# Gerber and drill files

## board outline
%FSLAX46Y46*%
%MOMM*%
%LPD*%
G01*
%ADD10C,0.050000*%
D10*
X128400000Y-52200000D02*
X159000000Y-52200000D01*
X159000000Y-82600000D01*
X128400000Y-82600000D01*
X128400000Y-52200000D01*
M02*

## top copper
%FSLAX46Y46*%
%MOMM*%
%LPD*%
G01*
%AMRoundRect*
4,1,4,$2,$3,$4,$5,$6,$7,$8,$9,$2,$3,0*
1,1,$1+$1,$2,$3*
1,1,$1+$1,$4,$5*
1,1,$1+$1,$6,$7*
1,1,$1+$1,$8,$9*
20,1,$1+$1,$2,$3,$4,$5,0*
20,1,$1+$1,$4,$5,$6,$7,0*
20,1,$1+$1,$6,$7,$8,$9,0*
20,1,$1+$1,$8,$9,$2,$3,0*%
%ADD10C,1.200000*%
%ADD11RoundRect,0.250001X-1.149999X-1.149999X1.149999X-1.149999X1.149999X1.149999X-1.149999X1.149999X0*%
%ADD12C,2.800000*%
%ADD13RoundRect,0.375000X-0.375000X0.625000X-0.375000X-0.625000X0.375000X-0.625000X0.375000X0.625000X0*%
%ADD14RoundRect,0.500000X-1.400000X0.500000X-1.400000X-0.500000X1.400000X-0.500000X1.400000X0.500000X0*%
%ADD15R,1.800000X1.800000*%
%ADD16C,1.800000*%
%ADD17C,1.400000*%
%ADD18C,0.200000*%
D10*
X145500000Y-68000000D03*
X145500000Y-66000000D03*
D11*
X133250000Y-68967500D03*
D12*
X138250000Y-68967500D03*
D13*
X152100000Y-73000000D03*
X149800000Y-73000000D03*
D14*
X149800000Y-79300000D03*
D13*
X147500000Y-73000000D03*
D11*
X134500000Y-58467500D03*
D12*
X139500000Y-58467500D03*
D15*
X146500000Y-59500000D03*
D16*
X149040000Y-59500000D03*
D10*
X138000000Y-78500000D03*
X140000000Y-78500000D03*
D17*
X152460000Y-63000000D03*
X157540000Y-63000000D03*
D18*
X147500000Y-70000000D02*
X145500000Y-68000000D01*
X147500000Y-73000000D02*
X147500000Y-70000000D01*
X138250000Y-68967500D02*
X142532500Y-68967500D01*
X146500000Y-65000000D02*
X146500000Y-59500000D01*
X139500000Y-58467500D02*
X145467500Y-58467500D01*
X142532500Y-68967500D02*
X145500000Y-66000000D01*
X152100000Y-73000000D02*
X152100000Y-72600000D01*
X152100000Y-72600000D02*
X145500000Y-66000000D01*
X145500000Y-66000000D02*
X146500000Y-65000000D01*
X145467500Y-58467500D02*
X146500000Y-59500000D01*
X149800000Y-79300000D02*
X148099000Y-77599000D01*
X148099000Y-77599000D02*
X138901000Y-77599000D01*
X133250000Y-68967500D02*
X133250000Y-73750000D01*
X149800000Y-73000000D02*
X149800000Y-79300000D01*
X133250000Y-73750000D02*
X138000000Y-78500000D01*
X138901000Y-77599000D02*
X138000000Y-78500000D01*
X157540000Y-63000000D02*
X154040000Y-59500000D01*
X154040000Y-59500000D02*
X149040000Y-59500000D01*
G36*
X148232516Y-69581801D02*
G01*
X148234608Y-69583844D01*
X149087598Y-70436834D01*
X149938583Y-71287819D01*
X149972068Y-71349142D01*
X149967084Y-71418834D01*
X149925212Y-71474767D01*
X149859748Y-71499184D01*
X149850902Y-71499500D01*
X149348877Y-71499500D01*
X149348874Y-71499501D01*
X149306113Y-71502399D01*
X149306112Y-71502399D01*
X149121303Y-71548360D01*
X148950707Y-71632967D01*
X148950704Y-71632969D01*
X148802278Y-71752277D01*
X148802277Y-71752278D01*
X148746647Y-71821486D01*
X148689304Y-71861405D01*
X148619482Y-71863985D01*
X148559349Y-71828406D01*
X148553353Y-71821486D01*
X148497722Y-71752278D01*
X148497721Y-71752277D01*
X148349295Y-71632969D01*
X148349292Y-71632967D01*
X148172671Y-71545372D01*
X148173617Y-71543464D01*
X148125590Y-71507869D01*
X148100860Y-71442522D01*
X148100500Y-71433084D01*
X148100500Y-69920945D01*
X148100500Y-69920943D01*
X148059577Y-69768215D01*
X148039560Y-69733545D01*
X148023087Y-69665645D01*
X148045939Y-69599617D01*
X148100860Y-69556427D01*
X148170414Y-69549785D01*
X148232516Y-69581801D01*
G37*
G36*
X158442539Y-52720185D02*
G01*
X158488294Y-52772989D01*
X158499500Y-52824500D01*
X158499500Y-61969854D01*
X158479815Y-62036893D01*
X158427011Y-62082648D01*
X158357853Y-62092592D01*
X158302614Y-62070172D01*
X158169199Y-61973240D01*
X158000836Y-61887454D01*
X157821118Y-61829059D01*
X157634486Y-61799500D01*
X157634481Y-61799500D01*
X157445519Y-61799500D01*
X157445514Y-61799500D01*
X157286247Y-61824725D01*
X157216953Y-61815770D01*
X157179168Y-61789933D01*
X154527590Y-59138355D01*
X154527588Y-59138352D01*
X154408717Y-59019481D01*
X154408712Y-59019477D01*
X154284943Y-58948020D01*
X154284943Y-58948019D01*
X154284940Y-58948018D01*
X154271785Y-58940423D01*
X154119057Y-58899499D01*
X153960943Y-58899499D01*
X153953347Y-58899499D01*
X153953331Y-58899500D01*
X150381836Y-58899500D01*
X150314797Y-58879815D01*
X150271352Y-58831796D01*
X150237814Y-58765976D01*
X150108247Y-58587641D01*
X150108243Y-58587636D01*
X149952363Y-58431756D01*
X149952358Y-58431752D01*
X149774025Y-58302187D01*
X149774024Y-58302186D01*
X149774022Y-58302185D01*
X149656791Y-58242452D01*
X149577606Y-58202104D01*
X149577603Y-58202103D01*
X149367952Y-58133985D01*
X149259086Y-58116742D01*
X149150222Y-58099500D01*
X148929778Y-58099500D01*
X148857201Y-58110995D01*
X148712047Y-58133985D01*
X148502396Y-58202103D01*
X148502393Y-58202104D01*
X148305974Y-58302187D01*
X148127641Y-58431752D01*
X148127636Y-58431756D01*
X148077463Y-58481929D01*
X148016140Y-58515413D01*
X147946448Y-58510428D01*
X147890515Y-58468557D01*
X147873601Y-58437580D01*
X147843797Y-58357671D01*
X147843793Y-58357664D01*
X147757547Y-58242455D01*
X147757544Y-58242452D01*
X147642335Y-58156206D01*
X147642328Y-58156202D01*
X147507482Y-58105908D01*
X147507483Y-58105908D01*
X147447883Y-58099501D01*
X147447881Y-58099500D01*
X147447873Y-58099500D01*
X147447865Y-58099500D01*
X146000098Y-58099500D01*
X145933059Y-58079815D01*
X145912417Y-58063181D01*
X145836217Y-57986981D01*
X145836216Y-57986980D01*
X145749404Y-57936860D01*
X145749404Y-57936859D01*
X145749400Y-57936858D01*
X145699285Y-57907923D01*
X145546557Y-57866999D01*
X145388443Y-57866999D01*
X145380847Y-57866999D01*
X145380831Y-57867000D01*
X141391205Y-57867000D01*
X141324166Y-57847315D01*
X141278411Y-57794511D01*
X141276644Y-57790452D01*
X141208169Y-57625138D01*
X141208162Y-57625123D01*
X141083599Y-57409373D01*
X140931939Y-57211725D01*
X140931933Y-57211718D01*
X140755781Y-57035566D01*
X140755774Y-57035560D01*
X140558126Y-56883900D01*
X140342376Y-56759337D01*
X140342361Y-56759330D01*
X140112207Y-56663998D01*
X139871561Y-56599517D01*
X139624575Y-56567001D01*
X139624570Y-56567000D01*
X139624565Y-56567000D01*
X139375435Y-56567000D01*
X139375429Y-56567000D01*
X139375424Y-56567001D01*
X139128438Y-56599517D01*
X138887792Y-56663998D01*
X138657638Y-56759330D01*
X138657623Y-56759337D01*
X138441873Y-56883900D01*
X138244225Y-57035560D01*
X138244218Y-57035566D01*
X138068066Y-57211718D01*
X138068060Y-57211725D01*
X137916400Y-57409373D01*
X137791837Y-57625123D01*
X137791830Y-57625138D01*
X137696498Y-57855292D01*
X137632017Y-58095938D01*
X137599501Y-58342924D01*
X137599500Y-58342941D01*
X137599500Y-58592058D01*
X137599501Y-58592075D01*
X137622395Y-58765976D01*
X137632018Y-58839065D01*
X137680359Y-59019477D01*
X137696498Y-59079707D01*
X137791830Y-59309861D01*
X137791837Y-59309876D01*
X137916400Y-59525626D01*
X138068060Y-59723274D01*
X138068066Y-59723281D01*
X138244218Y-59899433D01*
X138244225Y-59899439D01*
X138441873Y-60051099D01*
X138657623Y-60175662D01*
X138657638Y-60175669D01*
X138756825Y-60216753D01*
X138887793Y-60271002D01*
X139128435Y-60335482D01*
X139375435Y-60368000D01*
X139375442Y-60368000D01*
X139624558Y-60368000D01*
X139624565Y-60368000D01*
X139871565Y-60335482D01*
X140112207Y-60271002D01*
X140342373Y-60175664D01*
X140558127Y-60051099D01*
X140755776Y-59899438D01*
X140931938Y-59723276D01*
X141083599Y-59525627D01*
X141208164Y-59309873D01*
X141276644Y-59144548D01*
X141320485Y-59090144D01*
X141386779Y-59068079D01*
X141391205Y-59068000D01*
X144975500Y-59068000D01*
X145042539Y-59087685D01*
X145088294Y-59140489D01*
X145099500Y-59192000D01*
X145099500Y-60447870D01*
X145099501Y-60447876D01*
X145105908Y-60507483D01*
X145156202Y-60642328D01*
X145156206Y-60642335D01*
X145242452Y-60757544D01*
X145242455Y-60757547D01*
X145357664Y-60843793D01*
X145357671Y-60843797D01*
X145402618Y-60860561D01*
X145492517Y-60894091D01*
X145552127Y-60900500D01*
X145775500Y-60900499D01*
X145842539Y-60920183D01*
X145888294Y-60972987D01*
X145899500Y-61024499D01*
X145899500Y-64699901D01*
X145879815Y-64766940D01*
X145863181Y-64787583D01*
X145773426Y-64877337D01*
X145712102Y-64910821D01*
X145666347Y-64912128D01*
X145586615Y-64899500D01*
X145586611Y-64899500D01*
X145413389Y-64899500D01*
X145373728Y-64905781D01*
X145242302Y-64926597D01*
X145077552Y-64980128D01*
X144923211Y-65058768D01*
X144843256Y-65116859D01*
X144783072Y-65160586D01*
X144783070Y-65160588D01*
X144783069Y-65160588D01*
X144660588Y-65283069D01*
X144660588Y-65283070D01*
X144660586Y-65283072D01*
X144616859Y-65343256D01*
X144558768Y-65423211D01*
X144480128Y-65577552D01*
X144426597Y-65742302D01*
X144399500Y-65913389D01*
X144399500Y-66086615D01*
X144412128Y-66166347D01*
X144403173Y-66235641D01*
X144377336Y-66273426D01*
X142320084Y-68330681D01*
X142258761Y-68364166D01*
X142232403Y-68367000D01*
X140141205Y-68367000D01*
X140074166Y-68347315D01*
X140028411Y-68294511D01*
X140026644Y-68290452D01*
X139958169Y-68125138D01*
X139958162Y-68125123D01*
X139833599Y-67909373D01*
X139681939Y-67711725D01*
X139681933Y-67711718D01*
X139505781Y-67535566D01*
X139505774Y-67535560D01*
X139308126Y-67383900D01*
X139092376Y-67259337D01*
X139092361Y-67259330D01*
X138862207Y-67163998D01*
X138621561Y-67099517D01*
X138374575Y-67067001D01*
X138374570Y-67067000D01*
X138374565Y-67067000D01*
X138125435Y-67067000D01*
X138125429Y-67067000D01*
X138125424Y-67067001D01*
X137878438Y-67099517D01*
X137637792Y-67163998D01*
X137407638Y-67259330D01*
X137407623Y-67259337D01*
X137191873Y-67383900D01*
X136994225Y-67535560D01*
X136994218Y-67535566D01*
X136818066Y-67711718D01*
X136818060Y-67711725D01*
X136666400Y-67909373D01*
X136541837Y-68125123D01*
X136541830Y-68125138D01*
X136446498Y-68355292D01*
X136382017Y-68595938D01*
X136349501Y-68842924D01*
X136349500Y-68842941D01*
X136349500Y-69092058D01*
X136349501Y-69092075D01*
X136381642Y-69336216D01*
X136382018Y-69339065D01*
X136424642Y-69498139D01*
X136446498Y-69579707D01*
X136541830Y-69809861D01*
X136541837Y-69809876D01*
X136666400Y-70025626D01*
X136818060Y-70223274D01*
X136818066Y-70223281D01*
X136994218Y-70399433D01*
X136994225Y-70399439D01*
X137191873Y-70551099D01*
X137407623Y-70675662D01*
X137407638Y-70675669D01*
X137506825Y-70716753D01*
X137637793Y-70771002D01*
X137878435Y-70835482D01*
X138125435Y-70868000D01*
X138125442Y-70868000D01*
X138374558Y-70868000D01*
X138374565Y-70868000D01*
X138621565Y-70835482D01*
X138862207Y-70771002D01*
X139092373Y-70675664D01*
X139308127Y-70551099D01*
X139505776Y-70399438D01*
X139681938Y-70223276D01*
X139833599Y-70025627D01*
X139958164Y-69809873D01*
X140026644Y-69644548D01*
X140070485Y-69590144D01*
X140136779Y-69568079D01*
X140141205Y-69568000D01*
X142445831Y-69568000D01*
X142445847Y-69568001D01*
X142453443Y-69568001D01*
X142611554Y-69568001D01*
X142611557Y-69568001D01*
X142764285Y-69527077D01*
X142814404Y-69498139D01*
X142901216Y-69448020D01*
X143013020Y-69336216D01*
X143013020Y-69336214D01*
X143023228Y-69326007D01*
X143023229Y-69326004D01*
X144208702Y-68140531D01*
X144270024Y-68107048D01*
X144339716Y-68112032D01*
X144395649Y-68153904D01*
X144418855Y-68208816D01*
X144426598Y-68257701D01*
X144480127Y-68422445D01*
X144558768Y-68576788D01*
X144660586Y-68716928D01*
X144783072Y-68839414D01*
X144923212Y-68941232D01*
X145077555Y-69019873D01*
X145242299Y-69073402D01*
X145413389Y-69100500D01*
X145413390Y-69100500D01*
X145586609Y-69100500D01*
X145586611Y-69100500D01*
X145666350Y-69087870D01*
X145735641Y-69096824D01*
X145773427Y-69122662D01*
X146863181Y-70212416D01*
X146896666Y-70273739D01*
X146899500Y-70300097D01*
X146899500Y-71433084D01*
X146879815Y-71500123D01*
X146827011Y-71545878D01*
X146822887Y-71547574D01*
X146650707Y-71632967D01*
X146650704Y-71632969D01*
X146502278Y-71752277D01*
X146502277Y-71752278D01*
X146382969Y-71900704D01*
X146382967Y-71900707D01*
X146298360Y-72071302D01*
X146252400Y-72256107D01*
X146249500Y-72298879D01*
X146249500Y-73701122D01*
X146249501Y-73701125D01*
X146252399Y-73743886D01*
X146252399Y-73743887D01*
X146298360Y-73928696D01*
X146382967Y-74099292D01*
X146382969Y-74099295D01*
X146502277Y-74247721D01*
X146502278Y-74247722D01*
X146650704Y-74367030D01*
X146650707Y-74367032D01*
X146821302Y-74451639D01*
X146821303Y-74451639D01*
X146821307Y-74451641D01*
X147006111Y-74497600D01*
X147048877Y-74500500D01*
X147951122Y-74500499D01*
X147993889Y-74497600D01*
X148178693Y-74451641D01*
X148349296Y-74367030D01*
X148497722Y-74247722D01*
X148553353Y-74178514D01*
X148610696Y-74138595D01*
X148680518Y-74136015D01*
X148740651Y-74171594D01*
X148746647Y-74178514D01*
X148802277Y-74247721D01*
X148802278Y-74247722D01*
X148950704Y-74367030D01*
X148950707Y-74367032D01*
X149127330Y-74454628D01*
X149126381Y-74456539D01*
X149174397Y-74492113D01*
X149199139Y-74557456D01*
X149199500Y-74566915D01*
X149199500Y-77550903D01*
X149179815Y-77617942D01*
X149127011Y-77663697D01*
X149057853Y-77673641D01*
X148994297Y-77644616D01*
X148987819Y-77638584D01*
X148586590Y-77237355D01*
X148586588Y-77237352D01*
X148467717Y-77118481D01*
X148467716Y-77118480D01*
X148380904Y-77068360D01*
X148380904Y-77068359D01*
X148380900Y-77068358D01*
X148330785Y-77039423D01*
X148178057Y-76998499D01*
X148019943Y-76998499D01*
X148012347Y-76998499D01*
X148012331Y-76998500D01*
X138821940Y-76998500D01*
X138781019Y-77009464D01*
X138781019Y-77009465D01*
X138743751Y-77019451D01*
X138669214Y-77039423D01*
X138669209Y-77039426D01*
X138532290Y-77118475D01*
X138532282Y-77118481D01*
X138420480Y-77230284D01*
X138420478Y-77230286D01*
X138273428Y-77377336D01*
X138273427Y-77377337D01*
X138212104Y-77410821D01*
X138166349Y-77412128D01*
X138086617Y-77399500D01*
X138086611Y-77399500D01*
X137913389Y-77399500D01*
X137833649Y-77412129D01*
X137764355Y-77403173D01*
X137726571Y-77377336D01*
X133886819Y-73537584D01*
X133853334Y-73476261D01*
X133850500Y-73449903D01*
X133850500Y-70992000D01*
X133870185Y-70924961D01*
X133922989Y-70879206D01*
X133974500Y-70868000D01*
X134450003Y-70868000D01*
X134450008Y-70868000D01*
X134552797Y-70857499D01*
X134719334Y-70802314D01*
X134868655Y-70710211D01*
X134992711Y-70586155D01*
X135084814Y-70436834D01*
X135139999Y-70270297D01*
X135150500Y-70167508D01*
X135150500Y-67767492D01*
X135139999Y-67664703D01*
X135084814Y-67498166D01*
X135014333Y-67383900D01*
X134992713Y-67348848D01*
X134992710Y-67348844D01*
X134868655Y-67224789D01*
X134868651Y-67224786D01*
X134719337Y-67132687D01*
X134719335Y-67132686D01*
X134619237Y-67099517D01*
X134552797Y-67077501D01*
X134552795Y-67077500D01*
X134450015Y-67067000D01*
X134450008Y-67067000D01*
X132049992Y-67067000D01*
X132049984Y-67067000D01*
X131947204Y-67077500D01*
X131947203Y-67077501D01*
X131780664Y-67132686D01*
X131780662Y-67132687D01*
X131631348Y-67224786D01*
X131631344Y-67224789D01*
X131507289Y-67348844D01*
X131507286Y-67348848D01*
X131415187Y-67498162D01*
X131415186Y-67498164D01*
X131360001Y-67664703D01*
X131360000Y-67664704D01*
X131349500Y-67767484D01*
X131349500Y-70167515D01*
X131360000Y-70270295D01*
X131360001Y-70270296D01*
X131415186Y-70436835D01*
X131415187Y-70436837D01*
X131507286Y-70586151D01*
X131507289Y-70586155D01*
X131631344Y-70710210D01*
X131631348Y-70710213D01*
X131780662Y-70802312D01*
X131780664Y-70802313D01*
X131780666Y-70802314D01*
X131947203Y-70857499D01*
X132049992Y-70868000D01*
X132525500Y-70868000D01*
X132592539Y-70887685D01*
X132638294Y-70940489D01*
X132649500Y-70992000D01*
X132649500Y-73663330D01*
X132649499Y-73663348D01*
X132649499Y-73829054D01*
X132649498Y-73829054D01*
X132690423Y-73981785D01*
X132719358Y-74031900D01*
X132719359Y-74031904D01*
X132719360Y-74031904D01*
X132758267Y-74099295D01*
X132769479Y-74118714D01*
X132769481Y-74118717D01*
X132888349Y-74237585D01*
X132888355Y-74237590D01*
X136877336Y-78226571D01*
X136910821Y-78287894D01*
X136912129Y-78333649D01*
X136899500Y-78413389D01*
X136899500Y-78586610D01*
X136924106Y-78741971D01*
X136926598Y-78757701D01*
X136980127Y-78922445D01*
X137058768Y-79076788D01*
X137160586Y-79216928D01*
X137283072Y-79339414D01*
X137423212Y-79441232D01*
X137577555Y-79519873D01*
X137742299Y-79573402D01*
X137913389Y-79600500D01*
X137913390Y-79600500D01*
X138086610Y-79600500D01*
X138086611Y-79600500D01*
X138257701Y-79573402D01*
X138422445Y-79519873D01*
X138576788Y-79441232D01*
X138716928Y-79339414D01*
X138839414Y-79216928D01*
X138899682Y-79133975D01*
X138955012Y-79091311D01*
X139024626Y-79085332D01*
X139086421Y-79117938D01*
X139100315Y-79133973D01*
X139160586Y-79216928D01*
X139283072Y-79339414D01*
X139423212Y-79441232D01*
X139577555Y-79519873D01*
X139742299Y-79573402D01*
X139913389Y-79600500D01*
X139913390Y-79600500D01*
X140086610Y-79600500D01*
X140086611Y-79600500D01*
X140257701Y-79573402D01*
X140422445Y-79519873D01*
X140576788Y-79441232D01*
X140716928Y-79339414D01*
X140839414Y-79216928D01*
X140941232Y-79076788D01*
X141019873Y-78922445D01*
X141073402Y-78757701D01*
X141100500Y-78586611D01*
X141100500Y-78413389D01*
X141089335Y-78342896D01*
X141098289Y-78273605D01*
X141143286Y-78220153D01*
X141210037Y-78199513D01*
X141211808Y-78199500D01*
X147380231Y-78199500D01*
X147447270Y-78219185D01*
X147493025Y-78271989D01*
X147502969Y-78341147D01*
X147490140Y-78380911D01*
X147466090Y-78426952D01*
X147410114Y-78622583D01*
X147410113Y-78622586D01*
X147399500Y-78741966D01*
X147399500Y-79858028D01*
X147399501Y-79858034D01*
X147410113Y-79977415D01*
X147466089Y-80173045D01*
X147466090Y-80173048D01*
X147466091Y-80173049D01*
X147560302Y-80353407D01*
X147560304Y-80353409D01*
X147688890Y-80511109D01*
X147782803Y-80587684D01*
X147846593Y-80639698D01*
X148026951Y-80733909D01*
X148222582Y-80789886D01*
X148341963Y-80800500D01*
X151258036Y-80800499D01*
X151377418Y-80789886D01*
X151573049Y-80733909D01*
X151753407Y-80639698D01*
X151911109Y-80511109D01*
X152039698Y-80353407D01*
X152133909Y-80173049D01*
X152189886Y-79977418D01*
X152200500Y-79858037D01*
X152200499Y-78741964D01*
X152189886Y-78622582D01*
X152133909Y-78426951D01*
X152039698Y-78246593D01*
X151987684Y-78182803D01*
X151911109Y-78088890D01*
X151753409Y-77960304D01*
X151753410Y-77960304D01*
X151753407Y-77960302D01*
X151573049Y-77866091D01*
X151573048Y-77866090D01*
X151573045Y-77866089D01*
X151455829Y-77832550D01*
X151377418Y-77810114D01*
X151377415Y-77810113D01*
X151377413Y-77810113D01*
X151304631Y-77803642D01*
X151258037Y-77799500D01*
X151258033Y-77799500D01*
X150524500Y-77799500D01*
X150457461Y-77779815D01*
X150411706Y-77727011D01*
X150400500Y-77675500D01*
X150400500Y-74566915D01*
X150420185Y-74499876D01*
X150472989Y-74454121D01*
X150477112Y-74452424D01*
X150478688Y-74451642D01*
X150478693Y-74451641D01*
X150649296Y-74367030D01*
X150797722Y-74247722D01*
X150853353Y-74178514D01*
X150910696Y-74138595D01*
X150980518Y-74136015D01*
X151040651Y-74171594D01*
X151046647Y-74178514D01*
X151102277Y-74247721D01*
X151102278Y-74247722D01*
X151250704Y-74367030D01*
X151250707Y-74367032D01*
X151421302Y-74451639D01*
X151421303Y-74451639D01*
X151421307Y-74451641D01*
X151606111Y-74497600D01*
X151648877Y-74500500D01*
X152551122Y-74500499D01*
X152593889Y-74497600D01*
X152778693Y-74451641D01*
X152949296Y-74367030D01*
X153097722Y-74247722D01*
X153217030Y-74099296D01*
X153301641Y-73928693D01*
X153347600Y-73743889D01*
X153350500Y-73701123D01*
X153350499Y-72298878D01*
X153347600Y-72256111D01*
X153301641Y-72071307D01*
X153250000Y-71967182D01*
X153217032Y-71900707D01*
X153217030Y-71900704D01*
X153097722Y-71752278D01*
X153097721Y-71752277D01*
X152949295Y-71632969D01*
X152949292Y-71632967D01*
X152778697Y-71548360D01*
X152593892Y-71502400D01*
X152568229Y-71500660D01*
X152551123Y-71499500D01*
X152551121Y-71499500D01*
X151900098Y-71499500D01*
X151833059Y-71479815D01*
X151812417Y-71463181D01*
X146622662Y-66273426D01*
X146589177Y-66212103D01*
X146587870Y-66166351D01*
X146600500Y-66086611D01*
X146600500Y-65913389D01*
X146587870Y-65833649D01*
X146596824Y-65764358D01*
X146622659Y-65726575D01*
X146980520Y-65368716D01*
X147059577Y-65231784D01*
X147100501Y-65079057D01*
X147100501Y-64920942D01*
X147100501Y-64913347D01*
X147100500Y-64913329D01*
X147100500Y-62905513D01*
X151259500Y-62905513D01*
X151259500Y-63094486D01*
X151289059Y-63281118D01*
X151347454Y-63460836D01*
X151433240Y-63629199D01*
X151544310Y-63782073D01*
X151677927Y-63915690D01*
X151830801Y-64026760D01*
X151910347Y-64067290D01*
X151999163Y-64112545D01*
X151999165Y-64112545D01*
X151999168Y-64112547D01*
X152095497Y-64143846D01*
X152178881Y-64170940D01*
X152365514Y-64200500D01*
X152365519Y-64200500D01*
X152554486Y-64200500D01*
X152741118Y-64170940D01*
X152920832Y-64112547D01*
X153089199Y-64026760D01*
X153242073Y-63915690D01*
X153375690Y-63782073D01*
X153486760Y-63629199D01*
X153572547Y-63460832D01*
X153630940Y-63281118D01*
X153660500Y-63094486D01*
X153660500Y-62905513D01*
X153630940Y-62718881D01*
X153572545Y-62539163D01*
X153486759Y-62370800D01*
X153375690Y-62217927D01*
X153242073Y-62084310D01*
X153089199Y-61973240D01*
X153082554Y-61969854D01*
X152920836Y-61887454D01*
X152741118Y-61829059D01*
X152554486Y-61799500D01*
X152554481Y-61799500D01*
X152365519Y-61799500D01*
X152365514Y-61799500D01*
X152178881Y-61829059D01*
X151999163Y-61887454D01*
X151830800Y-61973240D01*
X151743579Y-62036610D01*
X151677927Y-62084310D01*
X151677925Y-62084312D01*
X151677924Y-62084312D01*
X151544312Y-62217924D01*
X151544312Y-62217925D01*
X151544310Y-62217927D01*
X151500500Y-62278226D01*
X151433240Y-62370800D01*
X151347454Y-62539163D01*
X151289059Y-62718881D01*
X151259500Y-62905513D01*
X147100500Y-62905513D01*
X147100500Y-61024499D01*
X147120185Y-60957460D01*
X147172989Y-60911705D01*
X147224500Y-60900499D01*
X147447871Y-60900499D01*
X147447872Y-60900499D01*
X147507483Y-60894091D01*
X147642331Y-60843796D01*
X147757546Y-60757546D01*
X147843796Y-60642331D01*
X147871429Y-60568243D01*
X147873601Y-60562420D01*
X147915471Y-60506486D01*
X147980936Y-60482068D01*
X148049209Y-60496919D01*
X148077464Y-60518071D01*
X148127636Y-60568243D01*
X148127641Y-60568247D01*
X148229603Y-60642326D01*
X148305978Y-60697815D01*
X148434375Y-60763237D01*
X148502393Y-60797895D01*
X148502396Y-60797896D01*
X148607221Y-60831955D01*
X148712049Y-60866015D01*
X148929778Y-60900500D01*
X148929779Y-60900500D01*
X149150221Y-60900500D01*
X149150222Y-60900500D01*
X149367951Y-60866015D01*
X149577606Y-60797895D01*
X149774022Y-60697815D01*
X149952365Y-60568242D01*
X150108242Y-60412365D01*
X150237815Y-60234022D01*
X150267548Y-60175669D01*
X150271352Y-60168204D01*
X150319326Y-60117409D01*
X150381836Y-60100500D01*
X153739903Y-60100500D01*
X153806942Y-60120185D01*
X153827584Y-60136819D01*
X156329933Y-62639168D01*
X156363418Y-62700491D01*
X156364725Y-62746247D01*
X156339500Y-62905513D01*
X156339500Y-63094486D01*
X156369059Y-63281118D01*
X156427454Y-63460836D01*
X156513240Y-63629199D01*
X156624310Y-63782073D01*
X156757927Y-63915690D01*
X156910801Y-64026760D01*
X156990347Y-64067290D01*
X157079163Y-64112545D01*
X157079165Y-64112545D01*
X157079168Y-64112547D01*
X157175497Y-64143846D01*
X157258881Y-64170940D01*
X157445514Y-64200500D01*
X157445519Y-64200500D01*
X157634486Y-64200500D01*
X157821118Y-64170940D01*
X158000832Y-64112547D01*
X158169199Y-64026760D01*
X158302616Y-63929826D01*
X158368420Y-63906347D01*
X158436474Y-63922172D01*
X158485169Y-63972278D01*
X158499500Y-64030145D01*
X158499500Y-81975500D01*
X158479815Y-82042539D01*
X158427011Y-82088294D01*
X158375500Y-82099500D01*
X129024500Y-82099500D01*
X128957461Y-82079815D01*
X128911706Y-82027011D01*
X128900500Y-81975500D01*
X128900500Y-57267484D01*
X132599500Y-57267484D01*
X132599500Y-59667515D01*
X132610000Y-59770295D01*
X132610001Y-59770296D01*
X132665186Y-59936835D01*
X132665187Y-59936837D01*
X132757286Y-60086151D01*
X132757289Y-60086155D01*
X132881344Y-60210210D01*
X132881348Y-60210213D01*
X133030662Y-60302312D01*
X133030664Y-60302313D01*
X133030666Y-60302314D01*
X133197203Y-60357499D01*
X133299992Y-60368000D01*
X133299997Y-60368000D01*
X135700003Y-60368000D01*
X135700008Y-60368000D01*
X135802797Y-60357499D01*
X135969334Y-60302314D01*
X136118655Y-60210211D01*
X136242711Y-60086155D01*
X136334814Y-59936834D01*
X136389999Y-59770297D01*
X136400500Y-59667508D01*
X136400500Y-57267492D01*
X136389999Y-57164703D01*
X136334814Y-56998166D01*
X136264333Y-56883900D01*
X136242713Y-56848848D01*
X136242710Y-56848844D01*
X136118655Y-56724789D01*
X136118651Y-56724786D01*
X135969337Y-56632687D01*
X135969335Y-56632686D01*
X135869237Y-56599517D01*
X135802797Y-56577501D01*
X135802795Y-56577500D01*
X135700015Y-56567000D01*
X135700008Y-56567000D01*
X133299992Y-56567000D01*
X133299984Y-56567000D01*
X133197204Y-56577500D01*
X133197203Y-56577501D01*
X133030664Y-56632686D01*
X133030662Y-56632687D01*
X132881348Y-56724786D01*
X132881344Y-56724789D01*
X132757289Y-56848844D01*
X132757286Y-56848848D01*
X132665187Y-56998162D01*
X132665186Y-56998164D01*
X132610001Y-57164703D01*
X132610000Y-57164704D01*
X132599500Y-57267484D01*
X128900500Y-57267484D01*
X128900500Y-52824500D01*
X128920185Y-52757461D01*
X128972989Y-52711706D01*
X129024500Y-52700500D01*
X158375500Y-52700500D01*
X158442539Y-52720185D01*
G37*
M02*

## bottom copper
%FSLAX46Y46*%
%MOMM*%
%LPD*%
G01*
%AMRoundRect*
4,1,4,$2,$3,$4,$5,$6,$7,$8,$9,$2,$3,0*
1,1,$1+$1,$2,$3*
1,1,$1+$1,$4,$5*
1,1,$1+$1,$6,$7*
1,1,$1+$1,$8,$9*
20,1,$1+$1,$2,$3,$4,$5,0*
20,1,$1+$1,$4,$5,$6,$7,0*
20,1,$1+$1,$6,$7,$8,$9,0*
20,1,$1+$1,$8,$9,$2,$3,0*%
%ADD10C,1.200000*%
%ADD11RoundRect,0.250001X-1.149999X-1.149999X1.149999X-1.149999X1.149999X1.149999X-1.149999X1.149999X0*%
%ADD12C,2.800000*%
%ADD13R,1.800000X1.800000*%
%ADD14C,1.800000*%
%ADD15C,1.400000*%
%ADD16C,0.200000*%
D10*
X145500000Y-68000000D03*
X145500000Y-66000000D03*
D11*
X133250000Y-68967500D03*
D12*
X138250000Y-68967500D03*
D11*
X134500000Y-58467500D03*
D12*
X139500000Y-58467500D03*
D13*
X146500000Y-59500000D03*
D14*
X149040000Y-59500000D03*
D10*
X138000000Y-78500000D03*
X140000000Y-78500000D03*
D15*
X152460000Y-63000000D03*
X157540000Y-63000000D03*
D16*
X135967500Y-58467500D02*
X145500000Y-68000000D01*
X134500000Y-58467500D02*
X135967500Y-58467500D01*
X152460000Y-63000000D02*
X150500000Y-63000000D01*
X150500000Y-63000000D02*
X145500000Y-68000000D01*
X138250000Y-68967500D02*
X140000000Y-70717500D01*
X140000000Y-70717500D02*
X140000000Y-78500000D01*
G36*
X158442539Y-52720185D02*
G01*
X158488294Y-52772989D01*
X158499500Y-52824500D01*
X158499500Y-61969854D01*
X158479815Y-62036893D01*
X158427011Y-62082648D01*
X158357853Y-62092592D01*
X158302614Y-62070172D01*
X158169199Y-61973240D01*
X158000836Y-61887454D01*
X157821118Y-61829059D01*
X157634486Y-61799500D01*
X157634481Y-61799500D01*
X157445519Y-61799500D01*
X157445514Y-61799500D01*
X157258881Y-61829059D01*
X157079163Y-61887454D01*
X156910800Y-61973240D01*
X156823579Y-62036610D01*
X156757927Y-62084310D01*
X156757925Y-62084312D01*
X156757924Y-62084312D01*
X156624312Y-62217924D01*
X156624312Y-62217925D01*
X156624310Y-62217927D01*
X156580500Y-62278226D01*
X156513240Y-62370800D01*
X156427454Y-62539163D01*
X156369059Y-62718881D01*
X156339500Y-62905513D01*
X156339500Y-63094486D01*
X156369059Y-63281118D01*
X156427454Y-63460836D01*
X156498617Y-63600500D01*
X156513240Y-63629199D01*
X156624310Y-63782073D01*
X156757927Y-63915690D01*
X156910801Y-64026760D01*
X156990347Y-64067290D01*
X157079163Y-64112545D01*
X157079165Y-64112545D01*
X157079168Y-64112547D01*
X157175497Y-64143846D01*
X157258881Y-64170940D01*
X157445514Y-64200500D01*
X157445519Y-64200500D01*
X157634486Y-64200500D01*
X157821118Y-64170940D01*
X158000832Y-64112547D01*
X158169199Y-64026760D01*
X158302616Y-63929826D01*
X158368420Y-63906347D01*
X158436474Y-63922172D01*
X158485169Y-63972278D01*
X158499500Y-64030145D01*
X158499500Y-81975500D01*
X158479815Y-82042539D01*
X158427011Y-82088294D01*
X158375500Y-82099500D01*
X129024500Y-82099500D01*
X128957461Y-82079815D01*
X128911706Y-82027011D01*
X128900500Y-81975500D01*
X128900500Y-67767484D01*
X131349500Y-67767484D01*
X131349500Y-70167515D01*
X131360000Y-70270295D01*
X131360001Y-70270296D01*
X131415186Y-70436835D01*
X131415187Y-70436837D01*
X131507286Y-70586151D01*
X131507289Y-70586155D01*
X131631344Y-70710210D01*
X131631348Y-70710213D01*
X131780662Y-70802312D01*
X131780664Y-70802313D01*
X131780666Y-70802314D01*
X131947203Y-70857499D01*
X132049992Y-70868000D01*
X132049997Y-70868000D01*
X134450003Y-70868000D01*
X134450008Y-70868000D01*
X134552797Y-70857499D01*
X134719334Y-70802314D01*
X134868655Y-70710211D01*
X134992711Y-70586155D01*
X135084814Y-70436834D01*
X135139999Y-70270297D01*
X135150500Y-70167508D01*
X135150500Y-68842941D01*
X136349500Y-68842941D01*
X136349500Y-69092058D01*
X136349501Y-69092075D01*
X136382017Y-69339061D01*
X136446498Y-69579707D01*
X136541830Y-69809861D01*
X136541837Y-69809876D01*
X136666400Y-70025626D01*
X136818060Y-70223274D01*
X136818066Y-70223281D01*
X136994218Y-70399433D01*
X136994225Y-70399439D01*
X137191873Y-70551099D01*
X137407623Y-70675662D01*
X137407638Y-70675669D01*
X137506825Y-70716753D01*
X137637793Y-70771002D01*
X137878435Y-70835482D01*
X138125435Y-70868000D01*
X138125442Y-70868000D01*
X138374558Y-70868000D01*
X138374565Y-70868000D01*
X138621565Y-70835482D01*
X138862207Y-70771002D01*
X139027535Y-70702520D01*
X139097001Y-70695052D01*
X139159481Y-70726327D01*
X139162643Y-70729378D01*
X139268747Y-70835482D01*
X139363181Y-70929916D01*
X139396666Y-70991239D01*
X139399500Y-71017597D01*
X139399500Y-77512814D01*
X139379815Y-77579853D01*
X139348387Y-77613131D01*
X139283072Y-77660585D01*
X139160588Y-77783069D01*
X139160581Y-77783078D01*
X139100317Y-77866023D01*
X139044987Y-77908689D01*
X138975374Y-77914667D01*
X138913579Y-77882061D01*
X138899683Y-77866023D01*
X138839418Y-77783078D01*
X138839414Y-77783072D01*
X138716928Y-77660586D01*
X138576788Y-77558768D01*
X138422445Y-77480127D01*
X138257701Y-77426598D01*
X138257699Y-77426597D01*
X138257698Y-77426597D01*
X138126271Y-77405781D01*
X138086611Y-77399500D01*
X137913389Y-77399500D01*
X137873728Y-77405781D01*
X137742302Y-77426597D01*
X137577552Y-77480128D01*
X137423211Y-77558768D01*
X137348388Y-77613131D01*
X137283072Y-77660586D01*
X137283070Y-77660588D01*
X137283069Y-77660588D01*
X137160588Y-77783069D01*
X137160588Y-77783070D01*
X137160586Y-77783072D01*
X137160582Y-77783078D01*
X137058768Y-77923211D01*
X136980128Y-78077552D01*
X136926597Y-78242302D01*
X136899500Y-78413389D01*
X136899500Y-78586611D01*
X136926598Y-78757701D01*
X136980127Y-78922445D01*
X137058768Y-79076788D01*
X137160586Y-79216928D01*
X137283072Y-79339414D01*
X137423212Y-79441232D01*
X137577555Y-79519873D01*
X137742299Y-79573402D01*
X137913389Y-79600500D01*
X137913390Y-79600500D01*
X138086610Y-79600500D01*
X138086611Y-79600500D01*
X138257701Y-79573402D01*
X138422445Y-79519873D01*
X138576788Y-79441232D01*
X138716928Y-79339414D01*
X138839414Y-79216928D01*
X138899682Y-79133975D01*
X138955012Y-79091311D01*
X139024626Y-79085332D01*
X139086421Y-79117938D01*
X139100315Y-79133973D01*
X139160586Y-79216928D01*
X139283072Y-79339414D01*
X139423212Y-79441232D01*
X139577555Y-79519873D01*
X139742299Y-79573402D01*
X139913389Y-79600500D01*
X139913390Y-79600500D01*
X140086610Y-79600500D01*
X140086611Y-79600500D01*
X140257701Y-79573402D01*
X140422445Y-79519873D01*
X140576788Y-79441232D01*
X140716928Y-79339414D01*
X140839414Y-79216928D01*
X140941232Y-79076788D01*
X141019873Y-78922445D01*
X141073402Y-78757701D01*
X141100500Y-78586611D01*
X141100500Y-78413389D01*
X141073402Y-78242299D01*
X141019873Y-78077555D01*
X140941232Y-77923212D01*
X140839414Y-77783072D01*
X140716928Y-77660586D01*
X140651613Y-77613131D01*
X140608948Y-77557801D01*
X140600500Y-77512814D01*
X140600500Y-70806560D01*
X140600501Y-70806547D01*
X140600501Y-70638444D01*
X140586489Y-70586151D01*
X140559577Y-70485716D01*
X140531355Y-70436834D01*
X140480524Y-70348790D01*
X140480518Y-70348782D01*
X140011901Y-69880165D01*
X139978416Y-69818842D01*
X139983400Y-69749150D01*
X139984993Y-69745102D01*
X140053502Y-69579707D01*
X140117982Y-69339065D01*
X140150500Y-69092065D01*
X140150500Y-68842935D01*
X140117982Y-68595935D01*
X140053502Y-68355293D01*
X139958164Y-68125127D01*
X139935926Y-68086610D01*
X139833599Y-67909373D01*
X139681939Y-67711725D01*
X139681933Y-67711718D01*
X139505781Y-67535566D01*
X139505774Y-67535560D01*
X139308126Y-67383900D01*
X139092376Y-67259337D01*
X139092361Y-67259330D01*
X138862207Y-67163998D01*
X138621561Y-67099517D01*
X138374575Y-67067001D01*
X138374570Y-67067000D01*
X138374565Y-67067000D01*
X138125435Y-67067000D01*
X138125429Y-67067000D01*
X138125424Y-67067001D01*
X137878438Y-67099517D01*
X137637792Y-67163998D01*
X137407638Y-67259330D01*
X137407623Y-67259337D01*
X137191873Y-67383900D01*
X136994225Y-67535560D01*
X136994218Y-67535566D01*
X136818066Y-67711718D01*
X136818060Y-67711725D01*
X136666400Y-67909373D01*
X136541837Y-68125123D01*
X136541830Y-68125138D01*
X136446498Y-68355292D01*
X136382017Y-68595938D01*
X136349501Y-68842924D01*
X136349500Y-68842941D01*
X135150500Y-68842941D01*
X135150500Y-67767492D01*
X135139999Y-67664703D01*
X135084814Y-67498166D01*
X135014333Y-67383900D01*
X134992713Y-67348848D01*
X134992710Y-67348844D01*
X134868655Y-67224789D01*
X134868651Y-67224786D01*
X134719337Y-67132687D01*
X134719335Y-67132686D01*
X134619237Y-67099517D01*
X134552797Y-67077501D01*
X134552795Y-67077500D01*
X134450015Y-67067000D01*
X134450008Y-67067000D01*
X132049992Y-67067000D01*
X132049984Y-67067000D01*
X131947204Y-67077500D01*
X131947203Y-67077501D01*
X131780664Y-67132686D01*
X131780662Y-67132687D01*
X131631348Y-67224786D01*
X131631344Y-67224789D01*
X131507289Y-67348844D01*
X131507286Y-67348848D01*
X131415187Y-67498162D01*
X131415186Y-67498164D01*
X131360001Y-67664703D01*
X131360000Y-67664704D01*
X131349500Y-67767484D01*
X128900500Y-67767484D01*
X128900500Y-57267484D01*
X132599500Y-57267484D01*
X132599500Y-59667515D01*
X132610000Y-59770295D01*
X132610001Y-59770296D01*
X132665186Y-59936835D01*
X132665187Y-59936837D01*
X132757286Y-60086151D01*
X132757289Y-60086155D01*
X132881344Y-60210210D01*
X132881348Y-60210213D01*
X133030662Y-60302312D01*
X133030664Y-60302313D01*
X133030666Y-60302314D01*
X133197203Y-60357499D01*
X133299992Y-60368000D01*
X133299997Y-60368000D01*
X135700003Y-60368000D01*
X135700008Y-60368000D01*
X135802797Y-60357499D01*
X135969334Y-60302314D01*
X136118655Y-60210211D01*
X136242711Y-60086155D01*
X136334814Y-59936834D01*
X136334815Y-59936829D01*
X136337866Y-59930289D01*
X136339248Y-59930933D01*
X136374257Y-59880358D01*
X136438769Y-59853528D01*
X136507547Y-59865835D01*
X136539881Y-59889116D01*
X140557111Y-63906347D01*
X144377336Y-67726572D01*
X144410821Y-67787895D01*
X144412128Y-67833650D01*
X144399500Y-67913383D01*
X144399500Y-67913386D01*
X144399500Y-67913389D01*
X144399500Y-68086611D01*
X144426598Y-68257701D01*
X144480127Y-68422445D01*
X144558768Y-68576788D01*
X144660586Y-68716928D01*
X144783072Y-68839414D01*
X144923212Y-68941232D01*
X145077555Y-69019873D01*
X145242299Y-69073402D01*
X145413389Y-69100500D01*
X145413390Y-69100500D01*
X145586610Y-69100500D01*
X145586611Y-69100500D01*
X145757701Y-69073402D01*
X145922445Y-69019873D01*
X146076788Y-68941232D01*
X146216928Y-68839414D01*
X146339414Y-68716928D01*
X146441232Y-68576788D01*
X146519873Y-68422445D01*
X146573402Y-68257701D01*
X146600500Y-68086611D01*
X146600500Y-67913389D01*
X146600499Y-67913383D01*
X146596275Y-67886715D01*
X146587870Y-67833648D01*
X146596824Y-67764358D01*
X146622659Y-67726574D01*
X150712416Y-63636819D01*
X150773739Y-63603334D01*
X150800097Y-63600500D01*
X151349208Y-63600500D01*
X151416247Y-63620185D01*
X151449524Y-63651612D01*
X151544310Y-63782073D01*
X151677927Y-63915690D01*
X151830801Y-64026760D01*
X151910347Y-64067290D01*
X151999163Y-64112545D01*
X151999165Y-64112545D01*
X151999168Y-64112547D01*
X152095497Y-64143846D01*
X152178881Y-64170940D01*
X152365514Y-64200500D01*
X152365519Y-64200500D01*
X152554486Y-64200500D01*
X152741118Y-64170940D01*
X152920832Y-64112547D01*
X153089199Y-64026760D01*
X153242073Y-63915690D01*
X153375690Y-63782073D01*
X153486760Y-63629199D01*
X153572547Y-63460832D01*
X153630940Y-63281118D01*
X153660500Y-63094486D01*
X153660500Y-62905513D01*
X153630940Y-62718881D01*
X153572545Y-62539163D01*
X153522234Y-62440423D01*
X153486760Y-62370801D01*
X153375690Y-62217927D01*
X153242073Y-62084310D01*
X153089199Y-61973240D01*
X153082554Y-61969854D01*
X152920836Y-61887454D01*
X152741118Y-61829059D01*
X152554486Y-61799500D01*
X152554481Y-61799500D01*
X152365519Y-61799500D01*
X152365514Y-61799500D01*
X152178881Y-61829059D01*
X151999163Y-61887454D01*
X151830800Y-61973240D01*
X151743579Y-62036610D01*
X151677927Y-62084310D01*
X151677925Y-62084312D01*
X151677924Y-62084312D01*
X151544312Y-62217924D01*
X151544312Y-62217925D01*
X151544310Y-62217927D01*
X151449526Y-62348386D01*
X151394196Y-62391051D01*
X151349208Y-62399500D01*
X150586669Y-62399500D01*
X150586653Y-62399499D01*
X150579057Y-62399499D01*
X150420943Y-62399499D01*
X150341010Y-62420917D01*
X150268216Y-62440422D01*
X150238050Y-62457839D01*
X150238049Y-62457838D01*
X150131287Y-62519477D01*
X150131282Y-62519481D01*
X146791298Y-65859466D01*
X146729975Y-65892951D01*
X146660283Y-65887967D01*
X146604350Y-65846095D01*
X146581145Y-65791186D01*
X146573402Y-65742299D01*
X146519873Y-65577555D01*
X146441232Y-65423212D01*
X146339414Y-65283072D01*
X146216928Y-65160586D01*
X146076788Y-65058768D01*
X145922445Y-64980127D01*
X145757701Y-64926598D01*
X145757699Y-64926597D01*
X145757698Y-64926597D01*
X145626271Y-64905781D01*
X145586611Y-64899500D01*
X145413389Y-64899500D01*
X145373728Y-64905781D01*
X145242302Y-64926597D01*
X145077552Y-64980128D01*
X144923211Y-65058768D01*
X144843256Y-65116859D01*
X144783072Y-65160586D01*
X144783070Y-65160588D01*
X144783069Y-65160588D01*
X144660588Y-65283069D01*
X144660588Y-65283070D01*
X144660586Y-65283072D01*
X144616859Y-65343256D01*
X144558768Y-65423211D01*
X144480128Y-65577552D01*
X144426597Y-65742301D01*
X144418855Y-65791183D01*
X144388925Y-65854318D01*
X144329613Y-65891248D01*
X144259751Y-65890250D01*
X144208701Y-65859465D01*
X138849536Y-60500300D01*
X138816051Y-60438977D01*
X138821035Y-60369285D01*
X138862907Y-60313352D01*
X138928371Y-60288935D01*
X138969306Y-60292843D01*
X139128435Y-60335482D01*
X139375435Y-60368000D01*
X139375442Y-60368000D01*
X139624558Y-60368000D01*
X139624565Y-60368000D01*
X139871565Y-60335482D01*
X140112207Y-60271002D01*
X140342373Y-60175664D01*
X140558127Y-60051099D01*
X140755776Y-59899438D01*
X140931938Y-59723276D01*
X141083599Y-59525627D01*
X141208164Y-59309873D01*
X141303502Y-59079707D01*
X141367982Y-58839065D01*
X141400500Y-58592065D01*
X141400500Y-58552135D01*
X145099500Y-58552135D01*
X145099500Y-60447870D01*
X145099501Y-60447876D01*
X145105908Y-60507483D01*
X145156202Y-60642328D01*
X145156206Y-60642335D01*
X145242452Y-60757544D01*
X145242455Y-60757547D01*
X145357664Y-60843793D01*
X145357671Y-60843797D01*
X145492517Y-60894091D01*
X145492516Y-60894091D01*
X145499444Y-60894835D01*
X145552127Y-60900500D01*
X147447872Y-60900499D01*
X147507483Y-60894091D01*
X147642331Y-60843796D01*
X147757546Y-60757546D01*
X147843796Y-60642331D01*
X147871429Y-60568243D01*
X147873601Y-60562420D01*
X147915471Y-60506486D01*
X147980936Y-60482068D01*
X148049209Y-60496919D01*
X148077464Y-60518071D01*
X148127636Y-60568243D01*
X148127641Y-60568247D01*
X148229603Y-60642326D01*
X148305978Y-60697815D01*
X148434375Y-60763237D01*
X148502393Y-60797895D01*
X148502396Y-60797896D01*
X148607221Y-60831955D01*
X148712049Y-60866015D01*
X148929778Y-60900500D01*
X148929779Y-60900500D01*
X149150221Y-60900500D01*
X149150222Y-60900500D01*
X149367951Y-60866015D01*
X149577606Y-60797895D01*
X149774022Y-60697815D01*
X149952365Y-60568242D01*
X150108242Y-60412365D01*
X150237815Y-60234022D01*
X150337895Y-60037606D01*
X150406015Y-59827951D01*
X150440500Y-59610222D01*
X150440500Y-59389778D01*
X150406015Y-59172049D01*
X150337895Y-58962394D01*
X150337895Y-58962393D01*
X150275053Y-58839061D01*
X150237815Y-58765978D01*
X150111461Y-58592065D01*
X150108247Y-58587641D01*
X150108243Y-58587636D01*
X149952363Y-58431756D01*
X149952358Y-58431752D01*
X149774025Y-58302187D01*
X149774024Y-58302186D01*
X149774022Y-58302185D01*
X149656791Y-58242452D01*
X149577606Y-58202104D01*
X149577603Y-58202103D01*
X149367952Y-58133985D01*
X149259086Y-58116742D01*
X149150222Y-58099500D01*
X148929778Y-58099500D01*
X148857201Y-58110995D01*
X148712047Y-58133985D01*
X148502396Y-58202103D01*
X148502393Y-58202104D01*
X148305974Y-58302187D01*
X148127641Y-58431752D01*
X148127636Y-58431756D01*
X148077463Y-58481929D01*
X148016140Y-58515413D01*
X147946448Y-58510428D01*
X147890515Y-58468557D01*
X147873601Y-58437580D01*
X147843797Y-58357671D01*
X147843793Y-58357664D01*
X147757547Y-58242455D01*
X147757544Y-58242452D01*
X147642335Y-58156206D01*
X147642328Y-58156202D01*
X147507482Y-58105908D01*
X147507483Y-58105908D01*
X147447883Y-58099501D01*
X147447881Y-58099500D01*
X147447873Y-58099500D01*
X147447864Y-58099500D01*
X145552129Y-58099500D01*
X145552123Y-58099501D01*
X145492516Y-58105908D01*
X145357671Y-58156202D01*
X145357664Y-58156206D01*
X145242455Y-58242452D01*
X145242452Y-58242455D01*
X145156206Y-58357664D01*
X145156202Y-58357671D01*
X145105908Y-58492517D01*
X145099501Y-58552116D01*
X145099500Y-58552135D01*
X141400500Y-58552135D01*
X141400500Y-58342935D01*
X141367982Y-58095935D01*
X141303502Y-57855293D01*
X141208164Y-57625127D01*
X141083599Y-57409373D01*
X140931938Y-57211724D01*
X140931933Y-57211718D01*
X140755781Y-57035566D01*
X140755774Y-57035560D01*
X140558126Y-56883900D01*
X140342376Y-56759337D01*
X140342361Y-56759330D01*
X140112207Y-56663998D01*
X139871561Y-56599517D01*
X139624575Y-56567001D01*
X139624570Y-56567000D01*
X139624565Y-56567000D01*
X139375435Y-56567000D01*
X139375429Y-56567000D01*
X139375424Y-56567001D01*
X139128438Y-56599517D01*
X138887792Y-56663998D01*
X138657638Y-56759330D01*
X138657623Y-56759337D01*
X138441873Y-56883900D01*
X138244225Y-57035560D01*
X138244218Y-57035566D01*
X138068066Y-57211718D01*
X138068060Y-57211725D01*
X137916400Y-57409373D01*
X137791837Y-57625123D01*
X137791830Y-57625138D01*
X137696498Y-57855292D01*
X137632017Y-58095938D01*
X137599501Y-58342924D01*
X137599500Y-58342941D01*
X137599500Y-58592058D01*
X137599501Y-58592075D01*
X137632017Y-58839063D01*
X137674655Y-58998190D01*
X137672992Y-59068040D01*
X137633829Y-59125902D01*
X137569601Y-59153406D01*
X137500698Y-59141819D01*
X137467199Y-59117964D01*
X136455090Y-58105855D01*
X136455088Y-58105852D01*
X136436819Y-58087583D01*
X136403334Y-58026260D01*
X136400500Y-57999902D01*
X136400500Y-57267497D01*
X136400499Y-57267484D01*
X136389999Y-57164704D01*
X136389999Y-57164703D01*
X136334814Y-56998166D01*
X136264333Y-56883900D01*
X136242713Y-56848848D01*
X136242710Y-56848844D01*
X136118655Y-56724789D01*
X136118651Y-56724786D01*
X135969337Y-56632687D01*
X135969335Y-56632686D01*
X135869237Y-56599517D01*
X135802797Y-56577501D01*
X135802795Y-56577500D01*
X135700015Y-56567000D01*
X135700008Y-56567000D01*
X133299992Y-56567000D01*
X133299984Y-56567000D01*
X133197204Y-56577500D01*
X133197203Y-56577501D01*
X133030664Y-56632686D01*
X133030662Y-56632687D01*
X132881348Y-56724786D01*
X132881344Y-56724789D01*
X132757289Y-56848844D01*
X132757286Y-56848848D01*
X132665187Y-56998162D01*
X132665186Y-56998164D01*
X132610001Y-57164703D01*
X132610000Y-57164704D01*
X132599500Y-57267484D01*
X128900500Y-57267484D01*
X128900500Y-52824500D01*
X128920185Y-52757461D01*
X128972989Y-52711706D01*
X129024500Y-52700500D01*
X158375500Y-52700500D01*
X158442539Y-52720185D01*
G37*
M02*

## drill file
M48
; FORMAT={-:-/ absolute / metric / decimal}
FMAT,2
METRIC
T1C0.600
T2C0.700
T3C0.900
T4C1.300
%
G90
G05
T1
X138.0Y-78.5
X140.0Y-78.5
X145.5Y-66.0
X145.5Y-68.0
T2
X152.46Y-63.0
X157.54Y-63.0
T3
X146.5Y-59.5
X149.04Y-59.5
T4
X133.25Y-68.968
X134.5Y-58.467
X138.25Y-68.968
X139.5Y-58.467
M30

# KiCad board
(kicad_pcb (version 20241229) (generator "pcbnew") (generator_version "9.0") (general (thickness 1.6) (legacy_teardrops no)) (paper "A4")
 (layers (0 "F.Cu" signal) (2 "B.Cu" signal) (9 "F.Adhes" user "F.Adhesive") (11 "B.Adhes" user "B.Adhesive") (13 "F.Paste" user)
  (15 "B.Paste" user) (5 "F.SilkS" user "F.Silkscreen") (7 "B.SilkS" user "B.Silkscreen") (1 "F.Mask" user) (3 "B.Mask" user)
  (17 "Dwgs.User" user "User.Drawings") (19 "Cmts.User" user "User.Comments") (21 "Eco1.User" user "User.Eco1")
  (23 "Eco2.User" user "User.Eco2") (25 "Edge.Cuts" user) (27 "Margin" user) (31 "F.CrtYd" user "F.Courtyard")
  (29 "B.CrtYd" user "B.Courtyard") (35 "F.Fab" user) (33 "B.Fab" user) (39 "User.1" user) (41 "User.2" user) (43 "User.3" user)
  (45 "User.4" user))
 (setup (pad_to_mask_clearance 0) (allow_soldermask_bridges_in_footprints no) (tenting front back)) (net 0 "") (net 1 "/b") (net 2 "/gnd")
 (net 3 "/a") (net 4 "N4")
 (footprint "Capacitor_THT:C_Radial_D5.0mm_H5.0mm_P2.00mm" (layer "F.Cu") (at 145.5 68 90)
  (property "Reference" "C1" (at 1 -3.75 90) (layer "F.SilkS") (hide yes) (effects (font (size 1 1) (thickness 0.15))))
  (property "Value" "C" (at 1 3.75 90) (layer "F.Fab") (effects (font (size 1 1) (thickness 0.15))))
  (pad "1" thru_hole circle (at 0 0 90) (size 1.2 1.2) (drill 0.6) (layers "*.Cu" "*.Mask") (remove_unused_layers no) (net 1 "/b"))
  (pad "2" thru_hole circle (at 2 0 90) (size 1.2 1.2) (drill 0.6) (layers "*.Cu" "*.Mask") (remove_unused_layers no) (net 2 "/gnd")))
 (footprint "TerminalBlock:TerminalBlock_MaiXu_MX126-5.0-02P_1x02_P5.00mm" (layer "F.Cu") (at 133.25 68.9675)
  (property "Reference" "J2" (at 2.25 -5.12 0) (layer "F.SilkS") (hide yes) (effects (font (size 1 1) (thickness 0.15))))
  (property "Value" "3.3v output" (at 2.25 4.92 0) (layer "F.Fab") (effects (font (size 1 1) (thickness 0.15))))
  (pad "1" thru_hole roundrect (at 0 0) (size 2.8 2.8) (drill 1.3) (layers "*.Cu" "*.Mask") (remove_unused_layers no)
   (roundrect_rratio 0.089286) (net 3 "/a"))
  (pad "2" thru_hole circle (at 5 0) (size 2.8 2.8) (drill 1.3) (layers "*.Cu" "*.Mask") (remove_unused_layers no) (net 2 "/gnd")))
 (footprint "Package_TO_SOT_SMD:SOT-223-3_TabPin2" (layer "F.Cu") (at 149.8 76.15 -90)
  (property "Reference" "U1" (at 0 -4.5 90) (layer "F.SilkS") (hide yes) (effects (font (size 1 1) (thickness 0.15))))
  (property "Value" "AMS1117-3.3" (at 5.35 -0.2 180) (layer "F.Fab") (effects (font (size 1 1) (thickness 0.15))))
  (pad "1" smd roundrect (at -3.15 -2.3 270) (size 2 1.5) (layers "F.Cu" "F.Mask" "F.Paste") (roundrect_rratio 0.25) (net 2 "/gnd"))
  (pad "2" smd roundrect (at -3.15 0 270) (size 2 1.5) (layers "F.Cu" "F.Mask" "F.Paste") (roundrect_rratio 0.25) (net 3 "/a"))
  (pad "2" smd roundrect (at 3.15 0 270) (size 2 3.8) (layers "F.Cu" "F.Mask" "F.Paste") (roundrect_rratio 0.25) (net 3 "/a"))
  (pad "3" smd roundrect (at -3.15 2.3 270) (size 2 1.5) (layers "F.Cu" "F.Mask" "F.Paste") (roundrect_rratio 0.25) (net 1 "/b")))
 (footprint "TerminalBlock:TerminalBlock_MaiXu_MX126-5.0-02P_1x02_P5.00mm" (layer "F.Cu") (at 134.5 58.4675)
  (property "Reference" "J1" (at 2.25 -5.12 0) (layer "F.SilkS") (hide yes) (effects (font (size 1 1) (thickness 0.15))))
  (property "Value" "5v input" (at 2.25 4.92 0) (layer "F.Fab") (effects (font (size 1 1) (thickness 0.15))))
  (pad "1" thru_hole roundrect (at 0 0) (size 2.8 2.8) (drill 1.3) (layers "*.Cu" "*.Mask") (remove_unused_layers no)
   (roundrect_rratio 0.089286) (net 1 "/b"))
  (pad "2" thru_hole circle (at 5 0) (size 2.8 2.8) (drill 1.3) (layers "*.Cu" "*.Mask") (remove_unused_layers no) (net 2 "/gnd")))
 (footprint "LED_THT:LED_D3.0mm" (layer "F.Cu") (at 146.5 59.5)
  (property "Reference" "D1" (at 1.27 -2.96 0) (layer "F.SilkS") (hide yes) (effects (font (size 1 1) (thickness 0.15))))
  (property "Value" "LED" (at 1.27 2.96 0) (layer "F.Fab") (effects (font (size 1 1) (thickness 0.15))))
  (pad "1" thru_hole rect (at 0 0) (size 1.8 1.8) (drill 0.9) (layers "*.Cu" "*.Mask") (remove_unused_layers no) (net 2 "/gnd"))
  (pad "2" thru_hole circle (at 2.54 0) (size 1.8 1.8) (drill 0.9) (layers "*.Cu" "*.Mask") (remove_unused_layers no) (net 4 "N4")))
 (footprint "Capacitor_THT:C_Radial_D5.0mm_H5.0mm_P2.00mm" (layer "F.Cu") (at 138 78.5)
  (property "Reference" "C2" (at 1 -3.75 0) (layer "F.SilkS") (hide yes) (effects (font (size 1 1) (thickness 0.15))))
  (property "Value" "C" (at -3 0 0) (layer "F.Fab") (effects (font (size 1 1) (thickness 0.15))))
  (pad "1" thru_hole circle (at 0 0) (size 1.2 1.2) (drill 0.6) (layers "*.Cu" "*.Mask") (remove_unused_layers no) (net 3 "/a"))
  (pad "2" thru_hole circle (at 2 0) (size 1.2 1.2) (drill 0.6) (layers "*.Cu" "*.Mask") (remove_unused_layers no) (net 2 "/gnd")))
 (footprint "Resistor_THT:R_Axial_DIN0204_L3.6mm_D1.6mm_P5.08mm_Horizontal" (layer "F.Cu") (at 152.46 63)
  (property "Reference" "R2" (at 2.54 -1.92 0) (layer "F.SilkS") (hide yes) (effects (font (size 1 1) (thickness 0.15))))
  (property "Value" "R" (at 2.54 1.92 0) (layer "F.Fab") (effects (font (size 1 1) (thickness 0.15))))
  (pad "1" thru_hole circle (at 0 0) (size 1.4 1.4) (drill 0.7) (layers "*.Cu" "*.Mask") (remove_unused_layers no) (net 1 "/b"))
  (pad "2" thru_hole circle (at 5.08 0) (size 1.4 1.4) (drill 0.7) (layers "*.Cu" "*.Mask") (remove_unused_layers no) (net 4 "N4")))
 (gr_rect (start 128.4 52.2) (end 159 82.6) (stroke (width 0.05) (type default)) (fill no) (layer "Edge.Cuts"))
 (segment (start 147.5 70) (end 145.5 68) (width 0.2) (layer "F.Cu") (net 1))
 (segment (start 147.5 73) (end 147.5 70) (width 0.2) (layer "F.Cu") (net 1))
 (segment (start 135.9675 58.4675) (end 145.5 68) (width 0.2) (layer "B.Cu") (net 1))
 (segment (start 134.5 58.4675) (end 135.9675 58.4675) (width 0.2) (layer "B.Cu") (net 1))
 (segment (start 152.46 63) (end 150.5 63) (width 0.2) (layer "B.Cu") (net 1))
 (segment (start 150.5 63) (end 145.5 68) (width 0.2) (layer "B.Cu") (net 1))
 (segment (start 138.25 68.9675) (end 142.5325 68.9675) (width 0.2) (layer "F.Cu") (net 2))
 (segment (start 146.5 65) (end 146.5 59.5) (width 0.2) (layer "F.Cu") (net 2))
 (segment (start 139.5 58.4675) (end 145.4675 58.4675) (width 0.2) (layer "F.Cu") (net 2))
 (segment (start 142.5325 68.9675) (end 145.5 66) (width 0.2) (layer "F.Cu") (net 2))
 (segment (start 152.1 73) (end 152.1 72.6) (width 0.2) (layer "F.Cu") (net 2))
 (segment (start 152.1 72.6) (end 145.5 66) (width 0.2) (layer "F.Cu") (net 2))
 (segment (start 145.5 66) (end 146.5 65) (width 0.2) (layer "F.Cu") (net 2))
 (segment (start 145.4675 58.4675) (end 146.5 59.5) (width 0.2) (layer "F.Cu") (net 2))
 (segment (start 138.25 68.9675) (end 140 70.7175) (width 0.2) (layer "B.Cu") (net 2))
 (segment (start 140 70.7175) (end 140 78.5) (width 0.2) (layer "B.Cu") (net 2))
 (segment (start 149.8 79.3) (end 148.099 77.599) (width 0.2) (layer "F.Cu") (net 3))
 (segment (start 148.099 77.599) (end 138.901 77.599) (width 0.2) (layer "F.Cu") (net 3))
 (segment (start 133.25 68.9675) (end 133.25 73.75) (width 0.2) (layer "F.Cu") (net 3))
 (segment (start 149.8 73) (end 149.8 79.3) (width 0.2) (layer "F.Cu") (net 3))
 (segment (start 133.25 73.75) (end 138 78.5) (width 0.2) (layer "F.Cu") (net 3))
 (segment (start 138.901 77.599) (end 138 78.5) (width 0.2) (layer "F.Cu") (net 3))
 (segment (start 157.54 63) (end 154.04 59.5) (width 0.2) (layer "F.Cu") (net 4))
 (segment (start 154.04 59.5) (end 149.04 59.5) (width 0.2) (layer "F.Cu") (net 4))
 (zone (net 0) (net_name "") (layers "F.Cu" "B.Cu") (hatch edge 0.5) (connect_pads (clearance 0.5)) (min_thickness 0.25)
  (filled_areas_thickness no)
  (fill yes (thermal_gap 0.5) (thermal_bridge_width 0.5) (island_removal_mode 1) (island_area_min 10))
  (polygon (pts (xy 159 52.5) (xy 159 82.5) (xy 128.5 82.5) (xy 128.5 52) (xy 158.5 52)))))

